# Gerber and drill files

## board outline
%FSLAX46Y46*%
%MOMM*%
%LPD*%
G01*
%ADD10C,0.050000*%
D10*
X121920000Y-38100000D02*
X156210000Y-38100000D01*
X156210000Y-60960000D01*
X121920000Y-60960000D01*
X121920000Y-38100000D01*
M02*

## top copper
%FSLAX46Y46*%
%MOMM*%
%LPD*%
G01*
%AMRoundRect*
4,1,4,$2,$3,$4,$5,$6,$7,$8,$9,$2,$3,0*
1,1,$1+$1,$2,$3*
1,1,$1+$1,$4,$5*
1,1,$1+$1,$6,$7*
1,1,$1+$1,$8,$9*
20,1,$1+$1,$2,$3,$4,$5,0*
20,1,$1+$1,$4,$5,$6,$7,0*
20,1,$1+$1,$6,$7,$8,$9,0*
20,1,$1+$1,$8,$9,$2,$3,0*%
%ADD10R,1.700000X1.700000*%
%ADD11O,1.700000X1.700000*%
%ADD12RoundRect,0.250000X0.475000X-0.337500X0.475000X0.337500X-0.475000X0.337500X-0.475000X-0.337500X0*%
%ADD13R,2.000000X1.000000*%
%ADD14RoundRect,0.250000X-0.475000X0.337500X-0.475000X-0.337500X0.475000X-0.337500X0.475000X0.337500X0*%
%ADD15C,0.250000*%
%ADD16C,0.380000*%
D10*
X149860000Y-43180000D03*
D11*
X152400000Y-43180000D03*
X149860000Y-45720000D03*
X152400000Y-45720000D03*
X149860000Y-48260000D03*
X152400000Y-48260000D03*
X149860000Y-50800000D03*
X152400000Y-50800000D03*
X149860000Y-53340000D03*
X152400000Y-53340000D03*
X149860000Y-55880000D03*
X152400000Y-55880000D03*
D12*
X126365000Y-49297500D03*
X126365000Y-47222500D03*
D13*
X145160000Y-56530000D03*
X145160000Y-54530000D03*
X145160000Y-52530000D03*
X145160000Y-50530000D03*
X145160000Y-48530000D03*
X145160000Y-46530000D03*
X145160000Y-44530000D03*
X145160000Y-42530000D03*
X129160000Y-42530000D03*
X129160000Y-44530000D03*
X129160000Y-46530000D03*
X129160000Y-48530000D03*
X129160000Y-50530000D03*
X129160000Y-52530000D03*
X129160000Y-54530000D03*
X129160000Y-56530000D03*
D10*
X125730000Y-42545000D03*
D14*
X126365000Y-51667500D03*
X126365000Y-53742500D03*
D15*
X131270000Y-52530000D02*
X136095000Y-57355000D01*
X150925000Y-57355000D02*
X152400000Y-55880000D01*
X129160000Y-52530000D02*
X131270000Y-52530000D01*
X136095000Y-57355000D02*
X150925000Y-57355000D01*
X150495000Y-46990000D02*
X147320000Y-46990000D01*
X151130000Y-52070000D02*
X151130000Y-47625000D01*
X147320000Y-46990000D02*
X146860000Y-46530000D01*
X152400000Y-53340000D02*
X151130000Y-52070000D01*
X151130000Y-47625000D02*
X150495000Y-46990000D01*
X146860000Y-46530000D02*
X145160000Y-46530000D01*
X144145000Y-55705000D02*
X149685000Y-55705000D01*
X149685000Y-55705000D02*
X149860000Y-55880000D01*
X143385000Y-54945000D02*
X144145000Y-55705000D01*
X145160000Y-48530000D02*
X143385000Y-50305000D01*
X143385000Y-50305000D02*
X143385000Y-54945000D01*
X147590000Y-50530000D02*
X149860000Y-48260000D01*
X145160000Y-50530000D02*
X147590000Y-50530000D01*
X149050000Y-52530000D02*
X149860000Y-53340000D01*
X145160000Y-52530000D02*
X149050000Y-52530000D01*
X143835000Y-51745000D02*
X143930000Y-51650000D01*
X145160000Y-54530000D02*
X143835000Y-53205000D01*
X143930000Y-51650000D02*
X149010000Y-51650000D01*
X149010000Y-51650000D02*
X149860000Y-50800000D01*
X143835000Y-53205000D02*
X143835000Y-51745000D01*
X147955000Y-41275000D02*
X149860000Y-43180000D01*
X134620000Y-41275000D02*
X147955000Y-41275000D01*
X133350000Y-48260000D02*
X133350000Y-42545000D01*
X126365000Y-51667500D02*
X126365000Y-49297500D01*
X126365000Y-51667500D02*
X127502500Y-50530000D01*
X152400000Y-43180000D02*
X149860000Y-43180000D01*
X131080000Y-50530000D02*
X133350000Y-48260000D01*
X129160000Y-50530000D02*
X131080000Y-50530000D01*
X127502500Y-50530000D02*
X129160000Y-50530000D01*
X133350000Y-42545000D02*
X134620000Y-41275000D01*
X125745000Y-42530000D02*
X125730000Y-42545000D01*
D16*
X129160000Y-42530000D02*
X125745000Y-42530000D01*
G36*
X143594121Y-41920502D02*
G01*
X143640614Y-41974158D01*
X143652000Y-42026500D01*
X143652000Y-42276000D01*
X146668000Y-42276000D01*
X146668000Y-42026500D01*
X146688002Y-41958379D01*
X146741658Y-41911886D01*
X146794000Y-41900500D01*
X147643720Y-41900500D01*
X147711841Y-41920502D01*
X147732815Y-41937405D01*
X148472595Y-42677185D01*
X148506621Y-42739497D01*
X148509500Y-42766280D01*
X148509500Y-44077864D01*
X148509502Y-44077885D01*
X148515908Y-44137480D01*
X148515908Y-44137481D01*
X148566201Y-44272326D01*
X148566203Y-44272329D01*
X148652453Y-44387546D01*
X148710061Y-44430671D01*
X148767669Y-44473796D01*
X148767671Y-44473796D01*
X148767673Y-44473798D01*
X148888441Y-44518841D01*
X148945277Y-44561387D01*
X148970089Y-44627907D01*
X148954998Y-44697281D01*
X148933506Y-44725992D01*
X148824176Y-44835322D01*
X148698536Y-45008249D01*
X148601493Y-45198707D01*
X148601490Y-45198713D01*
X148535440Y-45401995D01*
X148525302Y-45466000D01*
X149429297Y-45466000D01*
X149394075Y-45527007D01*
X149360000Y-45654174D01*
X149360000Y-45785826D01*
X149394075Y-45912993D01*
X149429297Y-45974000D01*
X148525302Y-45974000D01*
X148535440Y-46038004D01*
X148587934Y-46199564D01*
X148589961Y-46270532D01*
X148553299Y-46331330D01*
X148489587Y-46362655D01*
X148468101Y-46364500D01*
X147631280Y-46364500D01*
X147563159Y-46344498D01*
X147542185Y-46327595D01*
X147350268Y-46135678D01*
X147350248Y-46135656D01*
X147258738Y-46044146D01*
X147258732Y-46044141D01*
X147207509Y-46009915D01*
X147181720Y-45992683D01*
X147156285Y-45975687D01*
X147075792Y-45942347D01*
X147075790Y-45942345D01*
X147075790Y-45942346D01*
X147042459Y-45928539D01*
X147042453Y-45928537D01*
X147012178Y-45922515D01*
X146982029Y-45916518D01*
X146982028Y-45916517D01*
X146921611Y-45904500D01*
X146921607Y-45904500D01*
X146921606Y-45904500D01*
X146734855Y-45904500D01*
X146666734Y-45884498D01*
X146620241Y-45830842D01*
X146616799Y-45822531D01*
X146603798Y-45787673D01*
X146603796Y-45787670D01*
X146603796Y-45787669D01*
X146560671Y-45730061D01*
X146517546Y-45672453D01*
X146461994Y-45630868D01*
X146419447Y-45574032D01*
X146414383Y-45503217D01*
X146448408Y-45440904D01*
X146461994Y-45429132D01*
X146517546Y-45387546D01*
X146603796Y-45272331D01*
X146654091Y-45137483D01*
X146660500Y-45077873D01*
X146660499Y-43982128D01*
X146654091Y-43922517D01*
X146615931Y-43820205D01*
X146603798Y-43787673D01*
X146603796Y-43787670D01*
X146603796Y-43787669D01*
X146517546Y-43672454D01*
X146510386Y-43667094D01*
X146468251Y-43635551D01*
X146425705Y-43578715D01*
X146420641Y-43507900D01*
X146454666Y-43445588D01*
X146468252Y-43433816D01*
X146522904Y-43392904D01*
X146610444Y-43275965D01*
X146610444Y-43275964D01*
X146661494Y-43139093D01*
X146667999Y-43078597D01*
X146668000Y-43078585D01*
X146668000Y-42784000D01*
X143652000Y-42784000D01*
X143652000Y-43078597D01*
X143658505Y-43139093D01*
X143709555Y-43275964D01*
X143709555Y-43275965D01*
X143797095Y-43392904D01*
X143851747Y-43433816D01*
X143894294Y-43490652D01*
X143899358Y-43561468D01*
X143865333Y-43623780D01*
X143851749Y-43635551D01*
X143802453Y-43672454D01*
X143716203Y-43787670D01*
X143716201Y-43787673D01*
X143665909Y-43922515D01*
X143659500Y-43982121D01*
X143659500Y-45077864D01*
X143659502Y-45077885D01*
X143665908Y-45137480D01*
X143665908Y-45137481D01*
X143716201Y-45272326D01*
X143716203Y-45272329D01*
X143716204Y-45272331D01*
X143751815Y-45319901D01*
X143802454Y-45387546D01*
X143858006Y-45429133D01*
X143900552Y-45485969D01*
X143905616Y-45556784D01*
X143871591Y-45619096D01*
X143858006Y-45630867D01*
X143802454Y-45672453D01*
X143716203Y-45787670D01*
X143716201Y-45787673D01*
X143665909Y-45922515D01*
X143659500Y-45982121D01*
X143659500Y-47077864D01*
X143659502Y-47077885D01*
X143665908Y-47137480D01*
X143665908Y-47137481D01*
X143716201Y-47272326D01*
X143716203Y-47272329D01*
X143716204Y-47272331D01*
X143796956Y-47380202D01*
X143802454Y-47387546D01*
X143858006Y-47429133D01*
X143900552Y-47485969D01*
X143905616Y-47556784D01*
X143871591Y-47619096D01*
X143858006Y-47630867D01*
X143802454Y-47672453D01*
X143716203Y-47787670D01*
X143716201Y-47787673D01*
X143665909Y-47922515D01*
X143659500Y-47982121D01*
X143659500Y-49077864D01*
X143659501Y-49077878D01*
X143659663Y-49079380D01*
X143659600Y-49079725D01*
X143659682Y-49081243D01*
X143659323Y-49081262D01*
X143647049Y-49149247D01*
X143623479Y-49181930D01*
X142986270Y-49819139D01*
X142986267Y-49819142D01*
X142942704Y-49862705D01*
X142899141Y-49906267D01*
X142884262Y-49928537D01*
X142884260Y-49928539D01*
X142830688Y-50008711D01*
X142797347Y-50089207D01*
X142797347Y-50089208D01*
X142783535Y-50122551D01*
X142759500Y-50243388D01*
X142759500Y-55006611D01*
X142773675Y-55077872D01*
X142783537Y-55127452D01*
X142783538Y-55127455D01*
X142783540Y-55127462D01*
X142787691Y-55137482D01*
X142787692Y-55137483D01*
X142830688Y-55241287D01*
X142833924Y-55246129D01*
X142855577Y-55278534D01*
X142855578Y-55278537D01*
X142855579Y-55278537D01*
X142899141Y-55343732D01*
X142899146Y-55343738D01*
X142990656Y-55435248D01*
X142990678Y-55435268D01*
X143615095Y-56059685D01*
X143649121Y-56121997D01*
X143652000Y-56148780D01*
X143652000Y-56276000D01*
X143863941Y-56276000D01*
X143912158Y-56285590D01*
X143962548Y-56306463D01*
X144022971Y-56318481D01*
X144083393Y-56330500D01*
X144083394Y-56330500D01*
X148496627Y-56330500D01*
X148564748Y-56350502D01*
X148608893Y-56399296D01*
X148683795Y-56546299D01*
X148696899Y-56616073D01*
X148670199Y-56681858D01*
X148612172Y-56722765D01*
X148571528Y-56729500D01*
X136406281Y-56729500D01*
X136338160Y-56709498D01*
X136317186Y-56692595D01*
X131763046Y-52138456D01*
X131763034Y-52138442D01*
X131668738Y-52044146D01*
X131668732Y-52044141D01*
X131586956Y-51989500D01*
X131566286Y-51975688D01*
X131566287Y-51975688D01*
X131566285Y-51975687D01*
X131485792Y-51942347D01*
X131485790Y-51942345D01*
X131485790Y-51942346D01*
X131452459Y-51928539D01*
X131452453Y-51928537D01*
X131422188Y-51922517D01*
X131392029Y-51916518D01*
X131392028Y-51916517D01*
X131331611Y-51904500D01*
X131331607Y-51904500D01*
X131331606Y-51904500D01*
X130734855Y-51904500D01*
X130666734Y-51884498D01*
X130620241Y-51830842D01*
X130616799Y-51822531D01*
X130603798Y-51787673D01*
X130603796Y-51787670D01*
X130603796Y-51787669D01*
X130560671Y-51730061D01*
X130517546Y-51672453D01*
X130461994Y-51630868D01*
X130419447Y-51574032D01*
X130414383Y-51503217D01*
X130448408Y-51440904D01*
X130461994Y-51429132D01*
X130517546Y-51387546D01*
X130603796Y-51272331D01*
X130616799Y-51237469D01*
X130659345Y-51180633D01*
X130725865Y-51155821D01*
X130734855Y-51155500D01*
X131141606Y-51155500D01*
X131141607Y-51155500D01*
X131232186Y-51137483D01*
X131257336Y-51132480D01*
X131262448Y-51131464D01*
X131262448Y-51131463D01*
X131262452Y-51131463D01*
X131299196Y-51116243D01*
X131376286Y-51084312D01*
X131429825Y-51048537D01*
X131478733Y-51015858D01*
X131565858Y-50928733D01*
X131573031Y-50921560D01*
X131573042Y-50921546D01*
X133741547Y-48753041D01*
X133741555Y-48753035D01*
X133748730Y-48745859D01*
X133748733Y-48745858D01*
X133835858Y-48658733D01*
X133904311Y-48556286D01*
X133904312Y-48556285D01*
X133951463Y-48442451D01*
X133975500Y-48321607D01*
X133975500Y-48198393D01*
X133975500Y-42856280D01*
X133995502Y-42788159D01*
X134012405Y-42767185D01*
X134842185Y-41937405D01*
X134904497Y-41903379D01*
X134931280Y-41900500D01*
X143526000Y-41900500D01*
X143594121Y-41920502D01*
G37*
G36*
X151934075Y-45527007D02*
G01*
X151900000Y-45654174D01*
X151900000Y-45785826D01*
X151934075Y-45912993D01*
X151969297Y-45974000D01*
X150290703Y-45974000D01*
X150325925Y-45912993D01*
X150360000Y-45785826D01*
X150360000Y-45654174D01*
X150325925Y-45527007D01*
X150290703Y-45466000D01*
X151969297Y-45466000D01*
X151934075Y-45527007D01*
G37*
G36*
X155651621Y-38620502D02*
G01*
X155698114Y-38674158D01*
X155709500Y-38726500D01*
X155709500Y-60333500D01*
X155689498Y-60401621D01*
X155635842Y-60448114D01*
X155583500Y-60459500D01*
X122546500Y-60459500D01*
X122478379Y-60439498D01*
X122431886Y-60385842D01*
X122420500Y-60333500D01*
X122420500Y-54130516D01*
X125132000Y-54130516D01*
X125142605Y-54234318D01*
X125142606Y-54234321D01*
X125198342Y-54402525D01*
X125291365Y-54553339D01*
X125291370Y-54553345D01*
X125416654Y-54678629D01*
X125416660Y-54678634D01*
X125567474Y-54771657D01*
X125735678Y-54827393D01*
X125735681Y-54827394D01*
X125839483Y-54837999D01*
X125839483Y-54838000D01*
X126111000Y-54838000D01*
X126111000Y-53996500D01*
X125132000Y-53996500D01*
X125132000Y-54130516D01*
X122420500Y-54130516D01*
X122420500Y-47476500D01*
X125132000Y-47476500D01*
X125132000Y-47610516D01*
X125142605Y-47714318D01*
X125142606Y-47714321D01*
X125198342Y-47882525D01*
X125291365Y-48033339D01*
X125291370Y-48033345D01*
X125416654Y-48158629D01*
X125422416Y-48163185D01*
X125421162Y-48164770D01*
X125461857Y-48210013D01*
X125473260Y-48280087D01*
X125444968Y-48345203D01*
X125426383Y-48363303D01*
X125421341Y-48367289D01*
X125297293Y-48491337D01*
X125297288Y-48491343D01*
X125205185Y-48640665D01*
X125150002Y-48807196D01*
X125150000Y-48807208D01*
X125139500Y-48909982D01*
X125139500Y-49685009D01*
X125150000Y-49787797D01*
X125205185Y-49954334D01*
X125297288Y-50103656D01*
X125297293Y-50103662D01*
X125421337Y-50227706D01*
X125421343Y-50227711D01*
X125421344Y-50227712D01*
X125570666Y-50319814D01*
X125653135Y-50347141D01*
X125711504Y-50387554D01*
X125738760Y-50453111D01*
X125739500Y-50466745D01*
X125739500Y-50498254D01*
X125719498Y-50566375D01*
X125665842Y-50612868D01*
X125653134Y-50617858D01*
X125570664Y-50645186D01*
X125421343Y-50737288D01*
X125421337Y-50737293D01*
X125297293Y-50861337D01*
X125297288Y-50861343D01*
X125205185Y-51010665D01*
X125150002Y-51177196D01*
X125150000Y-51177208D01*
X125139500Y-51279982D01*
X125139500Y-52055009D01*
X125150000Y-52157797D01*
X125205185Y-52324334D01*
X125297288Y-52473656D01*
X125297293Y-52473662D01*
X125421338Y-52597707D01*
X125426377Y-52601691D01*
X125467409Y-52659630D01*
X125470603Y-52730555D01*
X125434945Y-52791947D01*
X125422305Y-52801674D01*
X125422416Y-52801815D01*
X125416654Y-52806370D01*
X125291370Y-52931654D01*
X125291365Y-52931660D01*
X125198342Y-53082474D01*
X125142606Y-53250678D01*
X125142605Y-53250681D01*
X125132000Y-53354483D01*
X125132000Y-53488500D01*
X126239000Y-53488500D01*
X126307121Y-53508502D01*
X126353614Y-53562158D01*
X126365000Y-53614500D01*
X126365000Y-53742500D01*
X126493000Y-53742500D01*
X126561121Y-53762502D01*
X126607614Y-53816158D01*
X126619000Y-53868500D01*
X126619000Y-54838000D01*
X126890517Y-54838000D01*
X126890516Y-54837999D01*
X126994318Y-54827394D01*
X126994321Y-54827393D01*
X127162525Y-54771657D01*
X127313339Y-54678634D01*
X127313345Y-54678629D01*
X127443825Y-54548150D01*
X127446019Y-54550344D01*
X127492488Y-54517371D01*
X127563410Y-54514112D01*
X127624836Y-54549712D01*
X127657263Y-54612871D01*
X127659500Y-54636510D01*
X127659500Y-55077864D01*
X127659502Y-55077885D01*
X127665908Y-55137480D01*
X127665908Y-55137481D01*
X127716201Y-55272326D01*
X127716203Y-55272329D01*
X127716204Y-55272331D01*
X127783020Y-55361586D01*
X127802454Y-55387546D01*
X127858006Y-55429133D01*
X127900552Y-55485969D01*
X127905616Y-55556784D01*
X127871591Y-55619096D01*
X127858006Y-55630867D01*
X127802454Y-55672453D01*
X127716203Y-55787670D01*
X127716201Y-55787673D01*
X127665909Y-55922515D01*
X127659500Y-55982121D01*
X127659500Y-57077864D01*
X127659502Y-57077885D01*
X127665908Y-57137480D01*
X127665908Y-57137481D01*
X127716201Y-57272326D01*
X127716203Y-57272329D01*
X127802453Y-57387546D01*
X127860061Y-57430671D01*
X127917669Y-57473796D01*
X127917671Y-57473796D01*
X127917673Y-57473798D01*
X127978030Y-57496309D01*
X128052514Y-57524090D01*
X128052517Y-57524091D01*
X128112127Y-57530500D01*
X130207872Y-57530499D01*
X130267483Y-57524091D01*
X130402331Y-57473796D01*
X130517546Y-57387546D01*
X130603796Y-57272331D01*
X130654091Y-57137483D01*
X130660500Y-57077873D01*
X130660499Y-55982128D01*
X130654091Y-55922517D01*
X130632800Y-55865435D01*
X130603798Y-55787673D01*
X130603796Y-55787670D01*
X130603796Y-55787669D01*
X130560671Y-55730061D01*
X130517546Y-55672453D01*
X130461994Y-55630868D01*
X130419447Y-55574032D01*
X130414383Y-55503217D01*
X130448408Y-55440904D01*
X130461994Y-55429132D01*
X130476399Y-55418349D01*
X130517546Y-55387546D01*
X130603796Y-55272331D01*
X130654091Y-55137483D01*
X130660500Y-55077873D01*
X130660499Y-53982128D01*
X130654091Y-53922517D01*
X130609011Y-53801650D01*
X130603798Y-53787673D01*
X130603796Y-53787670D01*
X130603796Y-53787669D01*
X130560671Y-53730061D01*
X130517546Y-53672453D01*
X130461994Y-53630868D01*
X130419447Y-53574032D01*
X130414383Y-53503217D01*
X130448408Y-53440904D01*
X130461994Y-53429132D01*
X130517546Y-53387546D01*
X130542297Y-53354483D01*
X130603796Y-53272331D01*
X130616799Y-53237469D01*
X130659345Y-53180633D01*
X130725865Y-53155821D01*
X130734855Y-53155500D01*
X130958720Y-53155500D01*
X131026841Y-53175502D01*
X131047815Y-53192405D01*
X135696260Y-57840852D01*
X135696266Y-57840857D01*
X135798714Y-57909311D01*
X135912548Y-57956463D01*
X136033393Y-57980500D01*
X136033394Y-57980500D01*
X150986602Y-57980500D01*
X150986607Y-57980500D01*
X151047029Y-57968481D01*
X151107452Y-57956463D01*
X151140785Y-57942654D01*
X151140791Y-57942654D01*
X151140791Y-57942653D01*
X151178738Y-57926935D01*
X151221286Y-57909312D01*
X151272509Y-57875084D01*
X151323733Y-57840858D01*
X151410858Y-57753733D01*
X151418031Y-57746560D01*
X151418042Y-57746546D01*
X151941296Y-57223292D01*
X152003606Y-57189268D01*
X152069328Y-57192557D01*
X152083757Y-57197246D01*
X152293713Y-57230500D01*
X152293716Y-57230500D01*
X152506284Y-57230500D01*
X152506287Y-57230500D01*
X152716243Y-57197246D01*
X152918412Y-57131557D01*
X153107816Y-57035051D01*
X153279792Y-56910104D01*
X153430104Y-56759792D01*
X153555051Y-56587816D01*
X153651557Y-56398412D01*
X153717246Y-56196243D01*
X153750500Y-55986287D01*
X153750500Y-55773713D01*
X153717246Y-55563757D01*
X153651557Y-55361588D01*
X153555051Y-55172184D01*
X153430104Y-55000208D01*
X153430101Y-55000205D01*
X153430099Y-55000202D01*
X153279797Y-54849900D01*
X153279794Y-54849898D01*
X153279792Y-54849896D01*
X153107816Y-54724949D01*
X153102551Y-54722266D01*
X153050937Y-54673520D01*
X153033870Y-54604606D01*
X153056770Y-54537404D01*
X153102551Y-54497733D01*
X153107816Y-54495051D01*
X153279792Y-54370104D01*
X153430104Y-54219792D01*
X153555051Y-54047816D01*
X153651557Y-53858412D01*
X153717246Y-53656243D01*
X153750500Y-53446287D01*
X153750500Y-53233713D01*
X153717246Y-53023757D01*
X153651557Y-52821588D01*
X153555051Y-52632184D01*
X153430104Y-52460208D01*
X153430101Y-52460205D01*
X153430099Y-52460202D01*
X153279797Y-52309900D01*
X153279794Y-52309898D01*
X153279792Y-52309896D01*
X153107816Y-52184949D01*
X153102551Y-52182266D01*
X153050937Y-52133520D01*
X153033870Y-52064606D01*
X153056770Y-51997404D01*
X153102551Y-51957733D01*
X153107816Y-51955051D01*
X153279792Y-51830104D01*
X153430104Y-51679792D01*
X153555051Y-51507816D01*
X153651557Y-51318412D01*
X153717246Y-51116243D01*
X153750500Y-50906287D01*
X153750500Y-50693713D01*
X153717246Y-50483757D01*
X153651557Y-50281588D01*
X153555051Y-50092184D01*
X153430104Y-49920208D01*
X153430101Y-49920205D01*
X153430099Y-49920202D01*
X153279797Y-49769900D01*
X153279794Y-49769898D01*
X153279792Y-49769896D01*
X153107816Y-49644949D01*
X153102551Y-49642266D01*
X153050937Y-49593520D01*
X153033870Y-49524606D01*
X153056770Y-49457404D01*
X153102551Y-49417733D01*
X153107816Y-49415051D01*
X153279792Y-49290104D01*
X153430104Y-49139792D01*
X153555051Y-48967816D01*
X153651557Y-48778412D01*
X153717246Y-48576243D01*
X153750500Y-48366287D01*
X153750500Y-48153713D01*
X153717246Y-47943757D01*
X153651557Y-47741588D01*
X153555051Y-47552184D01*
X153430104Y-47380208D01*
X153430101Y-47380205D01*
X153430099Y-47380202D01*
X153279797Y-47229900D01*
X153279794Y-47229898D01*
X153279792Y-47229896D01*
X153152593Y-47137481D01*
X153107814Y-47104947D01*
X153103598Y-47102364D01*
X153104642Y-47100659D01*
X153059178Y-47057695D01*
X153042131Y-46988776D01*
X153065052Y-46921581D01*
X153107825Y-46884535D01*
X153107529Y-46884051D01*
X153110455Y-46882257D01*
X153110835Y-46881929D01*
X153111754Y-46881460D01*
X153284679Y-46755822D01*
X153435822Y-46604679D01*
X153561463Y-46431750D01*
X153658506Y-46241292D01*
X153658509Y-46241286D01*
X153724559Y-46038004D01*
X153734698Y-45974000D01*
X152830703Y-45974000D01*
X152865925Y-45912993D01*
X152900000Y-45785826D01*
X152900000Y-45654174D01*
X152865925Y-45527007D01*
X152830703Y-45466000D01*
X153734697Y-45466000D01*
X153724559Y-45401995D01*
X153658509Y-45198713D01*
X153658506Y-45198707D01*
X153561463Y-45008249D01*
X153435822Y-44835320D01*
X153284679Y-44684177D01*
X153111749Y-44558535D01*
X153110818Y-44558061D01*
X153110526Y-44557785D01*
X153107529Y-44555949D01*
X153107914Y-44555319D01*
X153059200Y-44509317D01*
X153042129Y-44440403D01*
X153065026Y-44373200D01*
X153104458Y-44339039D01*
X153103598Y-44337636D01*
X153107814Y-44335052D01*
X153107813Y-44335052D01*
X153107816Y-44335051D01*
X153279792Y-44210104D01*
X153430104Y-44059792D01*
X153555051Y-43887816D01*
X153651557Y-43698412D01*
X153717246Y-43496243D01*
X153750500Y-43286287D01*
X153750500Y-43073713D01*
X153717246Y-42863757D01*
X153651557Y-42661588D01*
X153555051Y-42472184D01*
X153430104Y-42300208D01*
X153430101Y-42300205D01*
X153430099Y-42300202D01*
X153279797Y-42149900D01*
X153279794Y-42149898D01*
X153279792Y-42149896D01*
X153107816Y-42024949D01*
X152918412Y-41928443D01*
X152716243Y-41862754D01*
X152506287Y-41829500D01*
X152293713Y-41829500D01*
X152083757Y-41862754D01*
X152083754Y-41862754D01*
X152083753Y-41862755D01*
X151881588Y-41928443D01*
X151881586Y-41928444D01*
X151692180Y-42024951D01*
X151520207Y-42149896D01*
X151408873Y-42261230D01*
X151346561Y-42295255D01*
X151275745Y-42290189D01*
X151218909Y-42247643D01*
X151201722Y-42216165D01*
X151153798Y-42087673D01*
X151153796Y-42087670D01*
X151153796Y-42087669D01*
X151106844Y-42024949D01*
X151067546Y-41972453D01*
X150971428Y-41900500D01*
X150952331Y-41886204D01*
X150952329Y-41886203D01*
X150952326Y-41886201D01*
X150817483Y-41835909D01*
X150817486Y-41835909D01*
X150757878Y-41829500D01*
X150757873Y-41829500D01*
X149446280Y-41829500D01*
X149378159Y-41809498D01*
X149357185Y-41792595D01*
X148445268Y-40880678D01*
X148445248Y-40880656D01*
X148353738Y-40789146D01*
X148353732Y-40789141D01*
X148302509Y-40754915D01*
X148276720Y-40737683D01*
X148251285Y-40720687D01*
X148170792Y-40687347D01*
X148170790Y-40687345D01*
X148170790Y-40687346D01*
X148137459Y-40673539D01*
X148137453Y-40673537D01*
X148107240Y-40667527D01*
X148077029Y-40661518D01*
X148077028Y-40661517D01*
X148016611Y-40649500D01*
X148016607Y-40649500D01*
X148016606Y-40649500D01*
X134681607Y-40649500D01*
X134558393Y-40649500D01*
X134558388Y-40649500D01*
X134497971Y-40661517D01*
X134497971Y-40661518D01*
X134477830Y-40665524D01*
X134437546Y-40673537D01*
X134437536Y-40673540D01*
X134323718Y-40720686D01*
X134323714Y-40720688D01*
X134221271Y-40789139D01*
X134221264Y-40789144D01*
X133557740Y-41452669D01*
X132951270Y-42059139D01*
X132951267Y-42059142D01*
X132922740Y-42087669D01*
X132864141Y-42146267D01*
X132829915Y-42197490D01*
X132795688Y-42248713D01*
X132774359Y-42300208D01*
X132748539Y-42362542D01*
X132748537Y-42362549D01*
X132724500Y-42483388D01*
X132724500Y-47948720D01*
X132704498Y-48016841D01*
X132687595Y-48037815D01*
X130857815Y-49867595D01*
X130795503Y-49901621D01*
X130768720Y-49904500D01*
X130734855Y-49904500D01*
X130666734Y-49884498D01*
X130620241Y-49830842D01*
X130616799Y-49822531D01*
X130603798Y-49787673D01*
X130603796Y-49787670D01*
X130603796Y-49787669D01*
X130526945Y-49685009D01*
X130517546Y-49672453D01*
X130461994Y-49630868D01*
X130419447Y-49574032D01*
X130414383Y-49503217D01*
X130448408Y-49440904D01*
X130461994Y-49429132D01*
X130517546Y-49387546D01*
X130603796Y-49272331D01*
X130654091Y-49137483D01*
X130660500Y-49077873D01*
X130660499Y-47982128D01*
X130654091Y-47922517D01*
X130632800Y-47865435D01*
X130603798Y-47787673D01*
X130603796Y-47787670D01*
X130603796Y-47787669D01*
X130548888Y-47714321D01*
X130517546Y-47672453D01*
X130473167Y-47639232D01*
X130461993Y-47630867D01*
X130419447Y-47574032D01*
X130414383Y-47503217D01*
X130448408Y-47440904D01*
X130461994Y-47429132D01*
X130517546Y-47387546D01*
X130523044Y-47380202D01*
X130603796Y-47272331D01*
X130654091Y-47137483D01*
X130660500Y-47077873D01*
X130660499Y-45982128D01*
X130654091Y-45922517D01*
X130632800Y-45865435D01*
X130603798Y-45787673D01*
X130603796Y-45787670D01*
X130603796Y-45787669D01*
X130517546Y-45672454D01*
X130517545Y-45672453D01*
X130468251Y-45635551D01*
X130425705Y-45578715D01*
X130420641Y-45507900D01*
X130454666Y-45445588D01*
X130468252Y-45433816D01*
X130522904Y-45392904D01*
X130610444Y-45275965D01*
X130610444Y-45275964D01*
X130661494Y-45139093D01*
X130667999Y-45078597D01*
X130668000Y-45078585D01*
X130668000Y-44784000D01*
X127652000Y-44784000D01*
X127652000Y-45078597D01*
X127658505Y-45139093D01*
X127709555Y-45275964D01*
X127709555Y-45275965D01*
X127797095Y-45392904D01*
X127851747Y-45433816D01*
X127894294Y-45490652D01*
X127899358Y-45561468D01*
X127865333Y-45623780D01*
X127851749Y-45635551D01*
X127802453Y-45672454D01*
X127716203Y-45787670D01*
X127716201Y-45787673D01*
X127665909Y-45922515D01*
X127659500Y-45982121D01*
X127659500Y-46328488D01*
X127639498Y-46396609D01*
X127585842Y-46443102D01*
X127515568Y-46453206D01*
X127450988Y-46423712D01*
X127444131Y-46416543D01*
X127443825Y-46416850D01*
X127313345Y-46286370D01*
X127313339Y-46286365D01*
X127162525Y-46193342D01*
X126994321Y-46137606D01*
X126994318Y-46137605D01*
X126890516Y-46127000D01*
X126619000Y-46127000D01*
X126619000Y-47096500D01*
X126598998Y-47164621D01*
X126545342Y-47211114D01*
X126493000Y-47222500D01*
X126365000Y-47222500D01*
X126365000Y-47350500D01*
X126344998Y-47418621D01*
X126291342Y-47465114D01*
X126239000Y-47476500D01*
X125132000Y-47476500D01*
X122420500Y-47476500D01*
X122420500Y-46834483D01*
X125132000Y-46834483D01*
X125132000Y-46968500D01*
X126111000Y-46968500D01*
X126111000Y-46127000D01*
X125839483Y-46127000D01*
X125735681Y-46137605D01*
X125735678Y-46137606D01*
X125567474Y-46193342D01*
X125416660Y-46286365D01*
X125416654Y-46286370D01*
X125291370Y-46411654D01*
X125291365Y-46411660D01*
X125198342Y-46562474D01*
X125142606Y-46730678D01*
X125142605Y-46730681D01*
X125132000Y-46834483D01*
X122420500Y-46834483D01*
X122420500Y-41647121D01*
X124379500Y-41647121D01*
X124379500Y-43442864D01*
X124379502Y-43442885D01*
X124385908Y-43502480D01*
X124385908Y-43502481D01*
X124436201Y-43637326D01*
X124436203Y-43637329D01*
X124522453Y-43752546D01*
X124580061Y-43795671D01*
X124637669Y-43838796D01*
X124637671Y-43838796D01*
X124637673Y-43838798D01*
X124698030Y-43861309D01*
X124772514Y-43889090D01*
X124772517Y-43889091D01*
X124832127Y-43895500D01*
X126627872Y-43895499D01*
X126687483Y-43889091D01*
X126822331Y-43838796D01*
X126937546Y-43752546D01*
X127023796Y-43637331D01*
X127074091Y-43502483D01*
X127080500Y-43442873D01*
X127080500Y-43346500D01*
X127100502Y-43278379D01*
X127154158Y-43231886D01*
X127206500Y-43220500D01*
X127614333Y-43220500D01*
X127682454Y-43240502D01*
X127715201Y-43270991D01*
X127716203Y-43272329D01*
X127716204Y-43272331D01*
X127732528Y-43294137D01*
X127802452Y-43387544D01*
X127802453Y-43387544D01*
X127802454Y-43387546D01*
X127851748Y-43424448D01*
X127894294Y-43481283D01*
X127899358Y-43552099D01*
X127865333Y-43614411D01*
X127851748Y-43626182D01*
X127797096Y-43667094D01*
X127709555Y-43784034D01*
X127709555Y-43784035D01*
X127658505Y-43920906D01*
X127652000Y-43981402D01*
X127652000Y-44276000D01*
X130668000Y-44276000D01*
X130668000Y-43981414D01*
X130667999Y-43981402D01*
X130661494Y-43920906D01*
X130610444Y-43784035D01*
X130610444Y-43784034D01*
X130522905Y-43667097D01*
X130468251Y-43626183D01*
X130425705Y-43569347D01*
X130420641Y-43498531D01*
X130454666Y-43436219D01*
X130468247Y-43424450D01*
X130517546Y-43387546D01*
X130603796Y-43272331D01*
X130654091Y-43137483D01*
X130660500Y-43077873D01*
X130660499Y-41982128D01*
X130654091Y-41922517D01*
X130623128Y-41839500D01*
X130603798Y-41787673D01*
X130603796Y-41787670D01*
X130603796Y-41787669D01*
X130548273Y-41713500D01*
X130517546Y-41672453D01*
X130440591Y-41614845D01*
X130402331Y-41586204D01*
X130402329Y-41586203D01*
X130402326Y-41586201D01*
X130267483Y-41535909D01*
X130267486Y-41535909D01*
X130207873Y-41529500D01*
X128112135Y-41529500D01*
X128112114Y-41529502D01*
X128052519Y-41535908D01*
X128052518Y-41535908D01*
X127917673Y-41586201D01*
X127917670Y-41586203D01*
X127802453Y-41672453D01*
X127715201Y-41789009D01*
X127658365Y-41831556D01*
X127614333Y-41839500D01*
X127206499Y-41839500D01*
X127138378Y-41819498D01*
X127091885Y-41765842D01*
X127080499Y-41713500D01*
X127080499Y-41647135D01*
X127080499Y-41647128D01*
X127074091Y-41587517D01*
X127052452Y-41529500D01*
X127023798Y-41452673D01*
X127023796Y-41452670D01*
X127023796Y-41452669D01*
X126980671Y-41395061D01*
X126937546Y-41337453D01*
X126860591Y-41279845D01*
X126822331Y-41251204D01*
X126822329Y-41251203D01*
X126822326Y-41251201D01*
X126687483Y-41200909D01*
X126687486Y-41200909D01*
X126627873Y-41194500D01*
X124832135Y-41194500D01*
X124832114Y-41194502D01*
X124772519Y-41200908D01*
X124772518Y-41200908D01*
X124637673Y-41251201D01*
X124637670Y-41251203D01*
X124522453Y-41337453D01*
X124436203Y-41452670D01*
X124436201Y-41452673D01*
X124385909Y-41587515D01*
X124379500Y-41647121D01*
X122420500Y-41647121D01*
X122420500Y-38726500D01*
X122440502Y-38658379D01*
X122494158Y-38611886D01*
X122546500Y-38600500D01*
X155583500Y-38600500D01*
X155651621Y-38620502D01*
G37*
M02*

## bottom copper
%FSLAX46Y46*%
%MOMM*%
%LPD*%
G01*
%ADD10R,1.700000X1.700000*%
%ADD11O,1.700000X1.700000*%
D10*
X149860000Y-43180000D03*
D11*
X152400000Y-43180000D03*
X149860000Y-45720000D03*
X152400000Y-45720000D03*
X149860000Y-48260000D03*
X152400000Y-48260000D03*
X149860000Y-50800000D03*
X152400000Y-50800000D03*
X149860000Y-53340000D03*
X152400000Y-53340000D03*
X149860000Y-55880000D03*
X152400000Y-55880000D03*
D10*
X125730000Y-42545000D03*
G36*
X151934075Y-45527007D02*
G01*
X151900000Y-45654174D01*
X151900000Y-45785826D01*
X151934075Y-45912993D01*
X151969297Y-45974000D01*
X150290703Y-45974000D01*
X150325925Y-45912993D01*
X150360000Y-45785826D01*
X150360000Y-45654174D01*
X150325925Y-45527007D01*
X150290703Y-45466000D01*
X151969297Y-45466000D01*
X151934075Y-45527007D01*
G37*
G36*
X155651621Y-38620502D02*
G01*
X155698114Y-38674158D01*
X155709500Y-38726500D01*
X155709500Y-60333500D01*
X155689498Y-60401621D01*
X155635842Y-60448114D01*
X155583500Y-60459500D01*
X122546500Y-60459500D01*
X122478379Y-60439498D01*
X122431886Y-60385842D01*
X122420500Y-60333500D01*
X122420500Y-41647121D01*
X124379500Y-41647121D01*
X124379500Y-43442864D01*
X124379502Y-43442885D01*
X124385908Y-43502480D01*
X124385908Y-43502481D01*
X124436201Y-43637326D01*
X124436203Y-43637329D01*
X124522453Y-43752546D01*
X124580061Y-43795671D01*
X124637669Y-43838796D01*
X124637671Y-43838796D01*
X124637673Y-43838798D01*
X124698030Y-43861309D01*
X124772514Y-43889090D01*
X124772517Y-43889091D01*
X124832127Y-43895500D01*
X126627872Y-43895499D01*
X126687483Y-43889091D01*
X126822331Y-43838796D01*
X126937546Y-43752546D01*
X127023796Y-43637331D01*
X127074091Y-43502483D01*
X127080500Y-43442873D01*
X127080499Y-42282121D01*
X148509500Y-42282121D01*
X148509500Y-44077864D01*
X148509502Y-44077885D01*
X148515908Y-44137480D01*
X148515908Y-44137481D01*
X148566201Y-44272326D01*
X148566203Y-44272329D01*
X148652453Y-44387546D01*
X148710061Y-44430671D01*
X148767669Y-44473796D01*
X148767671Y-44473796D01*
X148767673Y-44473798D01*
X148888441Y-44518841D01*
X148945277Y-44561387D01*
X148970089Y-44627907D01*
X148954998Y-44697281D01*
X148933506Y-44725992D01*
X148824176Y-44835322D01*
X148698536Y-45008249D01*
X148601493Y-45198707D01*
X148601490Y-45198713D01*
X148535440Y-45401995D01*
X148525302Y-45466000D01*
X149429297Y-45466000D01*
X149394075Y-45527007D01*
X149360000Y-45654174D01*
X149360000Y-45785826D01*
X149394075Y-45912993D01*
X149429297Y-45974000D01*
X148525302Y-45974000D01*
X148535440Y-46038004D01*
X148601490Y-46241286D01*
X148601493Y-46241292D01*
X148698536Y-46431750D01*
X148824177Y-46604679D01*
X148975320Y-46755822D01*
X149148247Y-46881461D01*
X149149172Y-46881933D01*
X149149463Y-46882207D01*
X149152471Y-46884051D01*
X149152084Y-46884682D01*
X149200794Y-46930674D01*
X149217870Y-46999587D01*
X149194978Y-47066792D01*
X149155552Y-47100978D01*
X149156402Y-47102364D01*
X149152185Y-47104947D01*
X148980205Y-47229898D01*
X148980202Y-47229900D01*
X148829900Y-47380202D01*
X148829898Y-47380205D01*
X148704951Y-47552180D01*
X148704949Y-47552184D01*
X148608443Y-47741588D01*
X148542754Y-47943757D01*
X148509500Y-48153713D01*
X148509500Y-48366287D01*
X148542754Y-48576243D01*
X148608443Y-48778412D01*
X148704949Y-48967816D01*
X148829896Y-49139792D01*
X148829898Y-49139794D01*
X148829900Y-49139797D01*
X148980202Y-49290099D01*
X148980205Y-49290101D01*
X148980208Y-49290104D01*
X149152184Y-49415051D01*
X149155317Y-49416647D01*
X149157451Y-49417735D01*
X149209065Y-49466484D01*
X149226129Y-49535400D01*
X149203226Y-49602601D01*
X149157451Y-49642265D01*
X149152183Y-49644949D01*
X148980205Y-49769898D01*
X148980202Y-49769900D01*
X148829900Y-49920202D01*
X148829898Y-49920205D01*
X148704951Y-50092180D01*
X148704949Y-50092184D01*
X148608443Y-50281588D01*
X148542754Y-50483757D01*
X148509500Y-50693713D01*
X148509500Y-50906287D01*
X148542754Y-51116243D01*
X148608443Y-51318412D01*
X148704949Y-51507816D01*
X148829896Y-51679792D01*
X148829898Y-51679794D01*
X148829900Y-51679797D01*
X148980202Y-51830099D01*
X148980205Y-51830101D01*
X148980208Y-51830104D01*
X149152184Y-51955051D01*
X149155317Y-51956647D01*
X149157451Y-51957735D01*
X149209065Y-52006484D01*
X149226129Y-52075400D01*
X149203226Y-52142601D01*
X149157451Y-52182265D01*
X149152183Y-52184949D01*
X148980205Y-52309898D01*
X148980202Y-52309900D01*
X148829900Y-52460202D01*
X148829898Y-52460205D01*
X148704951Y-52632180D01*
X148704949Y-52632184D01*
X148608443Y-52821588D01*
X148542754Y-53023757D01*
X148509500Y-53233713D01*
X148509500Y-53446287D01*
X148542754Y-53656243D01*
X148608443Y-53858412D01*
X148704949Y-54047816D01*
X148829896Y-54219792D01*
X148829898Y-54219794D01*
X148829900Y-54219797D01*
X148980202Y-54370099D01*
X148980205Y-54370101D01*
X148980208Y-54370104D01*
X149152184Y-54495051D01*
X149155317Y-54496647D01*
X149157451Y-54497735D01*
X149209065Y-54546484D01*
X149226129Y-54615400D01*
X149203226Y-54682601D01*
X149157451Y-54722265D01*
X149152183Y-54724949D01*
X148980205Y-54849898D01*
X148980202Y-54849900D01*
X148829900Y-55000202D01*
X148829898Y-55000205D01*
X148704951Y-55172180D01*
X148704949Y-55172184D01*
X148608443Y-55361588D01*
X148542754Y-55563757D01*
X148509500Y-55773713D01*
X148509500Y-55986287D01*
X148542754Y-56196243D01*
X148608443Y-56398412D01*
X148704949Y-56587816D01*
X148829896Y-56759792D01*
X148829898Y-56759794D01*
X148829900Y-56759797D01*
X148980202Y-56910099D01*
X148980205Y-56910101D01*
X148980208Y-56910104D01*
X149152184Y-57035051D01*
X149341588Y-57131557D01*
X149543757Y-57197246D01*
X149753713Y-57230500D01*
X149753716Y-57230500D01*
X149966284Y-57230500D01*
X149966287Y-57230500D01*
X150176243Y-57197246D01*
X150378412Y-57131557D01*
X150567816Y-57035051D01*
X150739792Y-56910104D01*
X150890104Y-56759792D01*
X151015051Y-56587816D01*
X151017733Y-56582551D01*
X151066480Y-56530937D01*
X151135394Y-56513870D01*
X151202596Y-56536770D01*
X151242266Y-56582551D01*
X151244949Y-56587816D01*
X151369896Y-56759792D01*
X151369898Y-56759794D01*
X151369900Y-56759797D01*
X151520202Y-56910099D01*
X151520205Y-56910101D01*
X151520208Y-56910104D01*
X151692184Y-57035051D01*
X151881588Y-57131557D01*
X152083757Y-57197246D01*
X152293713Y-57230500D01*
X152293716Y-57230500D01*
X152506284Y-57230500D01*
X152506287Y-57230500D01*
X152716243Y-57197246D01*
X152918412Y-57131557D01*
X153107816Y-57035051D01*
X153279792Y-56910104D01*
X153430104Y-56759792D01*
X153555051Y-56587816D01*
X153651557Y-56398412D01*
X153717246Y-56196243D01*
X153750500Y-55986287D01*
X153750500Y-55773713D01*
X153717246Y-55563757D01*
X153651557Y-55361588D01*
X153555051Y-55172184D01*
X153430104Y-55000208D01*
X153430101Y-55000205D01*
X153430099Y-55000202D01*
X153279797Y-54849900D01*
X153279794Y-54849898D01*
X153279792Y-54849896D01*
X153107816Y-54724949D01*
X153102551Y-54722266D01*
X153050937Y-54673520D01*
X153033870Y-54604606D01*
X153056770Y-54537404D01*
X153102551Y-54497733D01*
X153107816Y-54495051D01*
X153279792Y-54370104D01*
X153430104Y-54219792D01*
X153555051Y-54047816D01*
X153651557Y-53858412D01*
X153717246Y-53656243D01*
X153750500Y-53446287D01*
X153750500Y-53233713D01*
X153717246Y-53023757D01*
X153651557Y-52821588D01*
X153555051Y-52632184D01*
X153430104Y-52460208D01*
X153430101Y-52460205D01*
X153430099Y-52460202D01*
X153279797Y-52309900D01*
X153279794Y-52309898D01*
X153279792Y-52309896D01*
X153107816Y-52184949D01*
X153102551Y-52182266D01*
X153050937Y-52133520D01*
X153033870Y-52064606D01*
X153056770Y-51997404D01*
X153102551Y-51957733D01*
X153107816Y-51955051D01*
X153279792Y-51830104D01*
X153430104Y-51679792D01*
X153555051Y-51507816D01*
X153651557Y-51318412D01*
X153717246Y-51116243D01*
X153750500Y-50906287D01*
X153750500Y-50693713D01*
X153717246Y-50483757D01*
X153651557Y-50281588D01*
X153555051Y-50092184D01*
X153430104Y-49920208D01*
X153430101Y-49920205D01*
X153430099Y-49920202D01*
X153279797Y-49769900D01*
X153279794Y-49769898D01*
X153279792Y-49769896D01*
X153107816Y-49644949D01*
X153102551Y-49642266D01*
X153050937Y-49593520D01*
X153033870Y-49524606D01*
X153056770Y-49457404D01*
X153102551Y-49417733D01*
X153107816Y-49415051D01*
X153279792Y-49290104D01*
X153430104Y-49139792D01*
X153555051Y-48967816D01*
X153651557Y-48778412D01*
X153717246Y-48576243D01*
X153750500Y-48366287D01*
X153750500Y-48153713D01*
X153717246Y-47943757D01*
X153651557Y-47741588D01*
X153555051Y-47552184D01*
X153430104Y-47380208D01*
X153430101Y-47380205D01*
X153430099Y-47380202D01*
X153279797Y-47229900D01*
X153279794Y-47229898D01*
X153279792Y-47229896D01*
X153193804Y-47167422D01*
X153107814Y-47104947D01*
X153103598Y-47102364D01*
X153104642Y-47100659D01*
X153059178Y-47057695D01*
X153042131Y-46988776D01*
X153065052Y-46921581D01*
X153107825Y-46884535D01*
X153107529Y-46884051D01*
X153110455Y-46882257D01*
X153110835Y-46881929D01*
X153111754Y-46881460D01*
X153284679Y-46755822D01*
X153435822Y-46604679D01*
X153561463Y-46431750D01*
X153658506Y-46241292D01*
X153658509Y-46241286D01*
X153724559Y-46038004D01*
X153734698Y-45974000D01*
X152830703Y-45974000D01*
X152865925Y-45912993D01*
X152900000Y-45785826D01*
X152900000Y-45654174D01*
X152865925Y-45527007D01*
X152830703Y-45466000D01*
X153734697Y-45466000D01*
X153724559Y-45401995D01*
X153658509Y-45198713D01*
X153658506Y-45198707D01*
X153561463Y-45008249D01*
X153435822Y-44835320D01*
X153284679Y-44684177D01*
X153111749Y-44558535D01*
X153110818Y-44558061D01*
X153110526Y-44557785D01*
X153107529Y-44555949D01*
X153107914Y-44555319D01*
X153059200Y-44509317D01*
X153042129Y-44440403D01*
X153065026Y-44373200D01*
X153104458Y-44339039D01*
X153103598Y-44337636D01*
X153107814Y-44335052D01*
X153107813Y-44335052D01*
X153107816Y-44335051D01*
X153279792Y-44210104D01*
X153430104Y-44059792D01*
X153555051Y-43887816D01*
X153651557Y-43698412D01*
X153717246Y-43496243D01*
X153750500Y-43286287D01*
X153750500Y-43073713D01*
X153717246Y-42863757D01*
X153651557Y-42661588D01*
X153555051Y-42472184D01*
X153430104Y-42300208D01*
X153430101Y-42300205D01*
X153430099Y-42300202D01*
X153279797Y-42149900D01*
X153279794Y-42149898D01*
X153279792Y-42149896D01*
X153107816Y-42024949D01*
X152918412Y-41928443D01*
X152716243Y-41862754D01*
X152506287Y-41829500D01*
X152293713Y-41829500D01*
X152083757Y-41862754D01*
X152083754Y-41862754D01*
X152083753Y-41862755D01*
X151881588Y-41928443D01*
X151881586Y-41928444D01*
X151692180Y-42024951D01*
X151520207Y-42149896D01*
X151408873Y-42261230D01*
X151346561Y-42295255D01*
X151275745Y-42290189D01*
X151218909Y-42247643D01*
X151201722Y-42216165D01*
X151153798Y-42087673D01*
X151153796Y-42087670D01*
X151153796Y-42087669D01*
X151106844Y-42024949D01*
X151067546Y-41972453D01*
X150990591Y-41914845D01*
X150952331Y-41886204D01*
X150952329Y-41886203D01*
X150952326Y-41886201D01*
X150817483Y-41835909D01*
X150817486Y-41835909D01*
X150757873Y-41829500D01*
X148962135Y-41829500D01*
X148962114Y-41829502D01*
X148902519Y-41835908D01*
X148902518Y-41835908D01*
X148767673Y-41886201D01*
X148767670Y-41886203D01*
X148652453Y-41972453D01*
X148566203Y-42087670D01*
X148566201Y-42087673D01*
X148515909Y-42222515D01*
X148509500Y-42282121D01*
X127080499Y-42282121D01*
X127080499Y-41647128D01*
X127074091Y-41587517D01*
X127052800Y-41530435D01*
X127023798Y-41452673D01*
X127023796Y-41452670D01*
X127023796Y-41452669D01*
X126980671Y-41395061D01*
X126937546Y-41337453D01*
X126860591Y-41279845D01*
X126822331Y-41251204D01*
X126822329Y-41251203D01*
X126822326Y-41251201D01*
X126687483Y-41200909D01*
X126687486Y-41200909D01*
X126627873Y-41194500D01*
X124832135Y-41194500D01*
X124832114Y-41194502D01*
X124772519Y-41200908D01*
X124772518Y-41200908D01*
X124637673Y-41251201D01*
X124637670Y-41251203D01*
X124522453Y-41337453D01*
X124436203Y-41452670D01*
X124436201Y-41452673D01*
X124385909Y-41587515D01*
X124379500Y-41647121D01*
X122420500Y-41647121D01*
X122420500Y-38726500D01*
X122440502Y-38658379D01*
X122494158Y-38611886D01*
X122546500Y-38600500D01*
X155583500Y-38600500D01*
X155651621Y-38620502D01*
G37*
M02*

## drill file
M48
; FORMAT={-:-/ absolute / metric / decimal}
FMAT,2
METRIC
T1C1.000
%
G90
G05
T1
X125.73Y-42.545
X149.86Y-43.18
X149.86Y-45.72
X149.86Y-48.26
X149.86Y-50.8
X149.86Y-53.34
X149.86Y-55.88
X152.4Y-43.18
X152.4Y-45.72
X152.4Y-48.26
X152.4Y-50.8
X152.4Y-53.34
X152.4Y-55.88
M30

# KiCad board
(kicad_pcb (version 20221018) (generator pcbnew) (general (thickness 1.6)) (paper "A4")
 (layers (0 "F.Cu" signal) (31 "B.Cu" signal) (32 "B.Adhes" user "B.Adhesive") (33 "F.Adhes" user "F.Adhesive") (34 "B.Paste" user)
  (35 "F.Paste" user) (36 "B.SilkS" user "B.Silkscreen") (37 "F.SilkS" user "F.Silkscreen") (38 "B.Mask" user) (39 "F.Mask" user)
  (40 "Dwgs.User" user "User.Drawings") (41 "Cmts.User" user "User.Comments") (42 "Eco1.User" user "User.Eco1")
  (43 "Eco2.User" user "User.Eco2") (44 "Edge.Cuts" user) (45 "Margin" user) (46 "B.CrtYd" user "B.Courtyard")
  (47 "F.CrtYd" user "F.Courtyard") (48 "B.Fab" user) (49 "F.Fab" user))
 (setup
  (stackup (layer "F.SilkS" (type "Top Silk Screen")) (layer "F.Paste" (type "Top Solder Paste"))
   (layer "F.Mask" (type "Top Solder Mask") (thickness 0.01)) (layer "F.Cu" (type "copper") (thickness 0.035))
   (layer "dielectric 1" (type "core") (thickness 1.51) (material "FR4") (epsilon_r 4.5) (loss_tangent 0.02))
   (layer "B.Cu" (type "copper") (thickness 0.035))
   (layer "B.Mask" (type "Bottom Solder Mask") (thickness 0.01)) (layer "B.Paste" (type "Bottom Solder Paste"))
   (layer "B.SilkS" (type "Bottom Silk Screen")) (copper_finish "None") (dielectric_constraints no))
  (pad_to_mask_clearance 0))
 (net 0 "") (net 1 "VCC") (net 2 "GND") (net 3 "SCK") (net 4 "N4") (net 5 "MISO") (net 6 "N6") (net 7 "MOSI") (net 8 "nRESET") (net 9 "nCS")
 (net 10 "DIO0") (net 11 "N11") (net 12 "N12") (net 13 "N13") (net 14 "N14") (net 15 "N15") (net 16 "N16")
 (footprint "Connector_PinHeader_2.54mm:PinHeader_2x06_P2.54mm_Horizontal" (layer "F.Cu") (at 149.86 43.18)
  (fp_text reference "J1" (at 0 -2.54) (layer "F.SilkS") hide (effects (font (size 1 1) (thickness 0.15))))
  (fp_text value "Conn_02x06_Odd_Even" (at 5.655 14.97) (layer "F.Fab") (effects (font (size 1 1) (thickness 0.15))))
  (pad "1" thru_hole rect (at 0 0) (size 1.7 1.7) (drill 1) (layers "*.Cu" "*.Mask") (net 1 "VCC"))
  (pad "2" thru_hole oval (at 2.54 0) (size 1.7 1.7) (drill 1) (layers "*.Cu" "*.Mask") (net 1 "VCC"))
  (pad "3" thru_hole oval (at 0 2.54) (size 1.7 1.7) (drill 1) (layers "*.Cu" "*.Mask") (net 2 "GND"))
  (pad "4" thru_hole oval (at 2.54 2.54) (size 1.7 1.7) (drill 1) (layers "*.Cu" "*.Mask") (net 2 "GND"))
  (pad "5" thru_hole oval (at 0 5.08) (size 1.7 1.7) (drill 1) (layers "*.Cu" "*.Mask") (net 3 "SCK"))
  (pad "6" thru_hole oval (at 2.54 5.08) (size 1.7 1.7) (drill 1) (layers "*.Cu" "*.Mask") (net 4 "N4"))
  (pad "7" thru_hole oval (at 0 7.62) (size 1.7 1.7) (drill 1) (layers "*.Cu" "*.Mask") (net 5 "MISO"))
  (pad "8" thru_hole oval (at 2.54 7.62) (size 1.7 1.7) (drill 1) (layers "*.Cu" "*.Mask") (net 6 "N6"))
  (pad "9" thru_hole oval (at 0 10.16) (size 1.7 1.7) (drill 1) (layers "*.Cu" "*.Mask") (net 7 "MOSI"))
  (pad "10" thru_hole oval (at 2.54 10.16) (size 1.7 1.7) (drill 1) (layers "*.Cu" "*.Mask") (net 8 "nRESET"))
  (pad "11" thru_hole oval (at 0 12.7) (size 1.7 1.7) (drill 1) (layers "*.Cu" "*.Mask") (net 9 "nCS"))
  (pad "12" thru_hole oval (at 2.54 12.7) (size 1.7 1.7) (drill 1) (layers "*.Cu" "*.Mask") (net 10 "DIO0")))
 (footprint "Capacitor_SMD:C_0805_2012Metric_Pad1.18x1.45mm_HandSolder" (layer "F.Cu") (at 126.365 48.26 90)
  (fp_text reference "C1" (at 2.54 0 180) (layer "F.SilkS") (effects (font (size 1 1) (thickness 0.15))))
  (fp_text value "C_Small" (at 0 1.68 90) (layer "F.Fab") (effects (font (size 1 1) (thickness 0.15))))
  (pad "1" smd roundrect (at -1.0375 0 90) (size 1.175 1.45) (layers "F.Cu" "F.Paste" "F.Mask") (roundrect_rratio 0.2127659574)
   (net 1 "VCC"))
  (pad "2" smd roundrect (at 1.0375 0 90) (size 1.175 1.45) (layers "F.Cu" "F.Paste" "F.Mask") (roundrect_rratio 0.2127659574) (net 2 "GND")))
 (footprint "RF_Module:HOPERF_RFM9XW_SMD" (layer "F.Cu") (at 137.16 49.53 180)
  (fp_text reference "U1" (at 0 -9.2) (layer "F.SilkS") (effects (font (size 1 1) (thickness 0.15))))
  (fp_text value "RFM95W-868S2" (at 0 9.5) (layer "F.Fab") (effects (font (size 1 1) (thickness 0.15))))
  (pad "1" smd rect (at -8 -7 180) (size 2 1) (layers "F.Cu" "F.Paste" "F.Mask") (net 2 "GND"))
  (pad "2" smd rect (at -8 -5 180) (size 2 1) (layers "F.Cu" "F.Paste" "F.Mask") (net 5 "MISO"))
  (pad "3" smd rect (at -8 -3 180) (size 2 1) (layers "F.Cu" "F.Paste" "F.Mask") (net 7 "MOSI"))
  (pad "4" smd rect (at -8 -1 180) (size 2 1) (layers "F.Cu" "F.Paste" "F.Mask") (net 3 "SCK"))
  (pad "5" smd rect (at -8 1 180) (size 2 1) (layers "F.Cu" "F.Paste" "F.Mask") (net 9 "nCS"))
  (pad "6" smd rect (at -8 3 180) (size 2 1) (layers "F.Cu" "F.Paste" "F.Mask") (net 8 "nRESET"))
  (pad "7" smd rect (at -8 5 180) (size 2 1) (layers "F.Cu" "F.Paste" "F.Mask") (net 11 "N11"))
  (pad "8" smd rect (at -8 7 180) (size 2 1) (layers "F.Cu" "F.Paste" "F.Mask") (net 2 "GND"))
  (pad "9" smd rect (at 8 7 180) (size 2 1) (layers "F.Cu" "F.Paste" "F.Mask") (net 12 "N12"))
  (pad "10" smd rect (at 8 5 180) (size 2 1) (layers "F.Cu" "F.Paste" "F.Mask") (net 2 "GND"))
  (pad "11" smd rect (at 8 3 180) (size 2 1) (layers "F.Cu" "F.Paste" "F.Mask") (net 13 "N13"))
  (pad "12" smd rect (at 8 1 180) (size 2 1) (layers "F.Cu" "F.Paste" "F.Mask") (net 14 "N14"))
  (pad "13" smd rect (at 8 -1 180) (size 2 1) (layers "F.Cu" "F.Paste" "F.Mask") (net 1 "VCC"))
  (pad "14" smd rect (at 8 -3 180) (size 2 1) (layers "F.Cu" "F.Paste" "F.Mask") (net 10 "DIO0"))
  (pad "15" smd rect (at 8 -5 180) (size 2 1) (layers "F.Cu" "F.Paste" "F.Mask") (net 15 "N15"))
  (pad "16" smd rect (at 8 -7 180) (size 2 1) (layers "F.Cu" "F.Paste" "F.Mask") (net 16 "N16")))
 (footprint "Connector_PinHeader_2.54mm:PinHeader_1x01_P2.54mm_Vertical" (layer "F.Cu") (at 125.73 42.545)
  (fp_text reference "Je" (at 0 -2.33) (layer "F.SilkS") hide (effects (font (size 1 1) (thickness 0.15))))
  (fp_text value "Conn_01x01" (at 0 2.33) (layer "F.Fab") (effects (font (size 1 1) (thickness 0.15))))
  (pad "1" thru_hole rect (at 0 0) (size 1.7 1.7) (drill 1) (layers "*.Cu" "*.Mask") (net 12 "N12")))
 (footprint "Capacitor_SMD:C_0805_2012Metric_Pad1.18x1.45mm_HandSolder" (layer "F.Cu") (at 126.365 52.705 -90)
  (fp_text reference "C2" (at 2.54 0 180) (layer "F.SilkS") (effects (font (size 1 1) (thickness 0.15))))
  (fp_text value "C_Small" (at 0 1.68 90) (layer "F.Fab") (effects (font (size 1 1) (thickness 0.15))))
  (pad "1" smd roundrect (at -1.0375 0 270) (size 1.175 1.45) (layers "F.Cu" "F.Paste" "F.Mask") (roundrect_rratio 0.2127659574)
   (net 1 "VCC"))
  (pad "2" smd roundrect (at 1.0375 0 270) (size 1.175 1.45) (layers "F.Cu" "F.Paste" "F.Mask") (roundrect_rratio 0.2127659574)
   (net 2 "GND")))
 (gr_rect (start 121.92 38.1) (end 156.21 60.96) (stroke (width 0.05) (type solid)) (fill none) (layer "Edge.Cuts"))
 (segment (start 131.27 52.53) (end 136.095 57.355) (width 0.25) (layer "F.Cu") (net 10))
 (segment (start 150.925 57.355) (end 152.4 55.88) (width 0.25) (layer "F.Cu") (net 10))
 (segment (start 129.16 52.53) (end 131.27 52.53) (width 0.25) (layer "F.Cu") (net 10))
 (segment (start 136.095 57.355) (end 150.925 57.355) (width 0.25) (layer "F.Cu") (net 10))
 (segment (start 150.495 46.99) (end 147.32 46.99) (width 0.25) (layer "F.Cu") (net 8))
 (segment (start 151.13 52.07) (end 151.13 47.625) (width 0.25) (layer "F.Cu") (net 8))
 (segment (start 147.32 46.99) (end 146.86 46.53) (width 0.25) (layer "F.Cu") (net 8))
 (segment (start 152.4 53.34) (end 151.13 52.07) (width 0.25) (layer "F.Cu") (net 8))
 (segment (start 151.13 47.625) (end 150.495 46.99) (width 0.25) (layer "F.Cu") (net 8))
 (segment (start 146.86 46.53) (end 145.16 46.53) (width 0.25) (layer "F.Cu") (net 8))
 (segment (start 144.145 55.705) (end 149.685 55.705) (width 0.25) (layer "F.Cu") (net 9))
 (segment (start 149.685 55.705) (end 149.86 55.88) (width 0.25) (layer "F.Cu") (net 9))
 (segment (start 143.385 54.945) (end 144.145 55.705) (width 0.25) (layer "F.Cu") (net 9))
 (segment (start 145.16 48.53) (end 143.385 50.305) (width 0.25) (layer "F.Cu") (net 9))
 (segment (start 143.385 50.305) (end 143.385 54.945) (width 0.25) (layer "F.Cu") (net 9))
 (segment (start 147.59 50.53) (end 149.86 48.26) (width 0.25) (layer "F.Cu") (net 3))
 (segment (start 145.16 50.53) (end 147.59 50.53) (width 0.25) (layer "F.Cu") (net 3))
 (segment (start 149.05 52.53) (end 149.86 53.34) (width 0.25) (layer "F.Cu") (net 7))
 (segment (start 145.16 52.53) (end 149.05 52.53) (width 0.25) (layer "F.Cu") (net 7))
 (segment (start 143.835 51.745) (end 143.93 51.65) (width 0.25) (layer "F.Cu") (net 5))
 (segment (start 145.16 54.53) (end 143.835 53.205) (width 0.25) (layer "F.Cu") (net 5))
 (segment (start 143.93 51.65) (end 149.01 51.65) (width 0.25) (layer "F.Cu") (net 5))
 (segment (start 149.01 51.65) (end 149.86 50.8) (width 0.25) (layer "F.Cu") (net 5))
 (segment (start 143.835 53.205) (end 143.835 51.745) (width 0.25) (layer "F.Cu") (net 5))
 (segment (start 147.955 41.275) (end 149.86 43.18) (width 0.25) (layer "F.Cu") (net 1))
 (segment (start 134.62 41.275) (end 147.955 41.275) (width 0.25) (layer "F.Cu") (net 1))
 (segment (start 133.35 48.26) (end 133.35 42.545) (width 0.25) (layer "F.Cu") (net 1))
 (segment (start 126.365 51.6675) (end 126.365 49.2975) (width 0.25) (layer "F.Cu") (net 1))
 (segment (start 126.365 51.6675) (end 127.5025 50.53) (width 0.25) (layer "F.Cu") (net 1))
 (segment (start 152.4 43.18) (end 149.86 43.18) (width 0.25) (layer "F.Cu") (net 1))
 (segment (start 131.08 50.53) (end 133.35 48.26) (width 0.25) (layer "F.Cu") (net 1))
 (segment (start 129.16 50.53) (end 131.08 50.53) (width 0.25) (layer "F.Cu") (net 1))
 (segment (start 127.5025 50.53) (end 129.16 50.53) (width 0.25) (layer "F.Cu") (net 1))
 (segment (start 133.35 42.545) (end 134.62 41.275) (width 0.25) (layer "F.Cu") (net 1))
 (segment (start 125.745 42.53) (end 125.73 42.545) (width 0.25) (layer "F.Cu") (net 12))
 (segment (start 129.16 42.53) (end 125.745 42.53) (width 0.38) (layer "F.Cu") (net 12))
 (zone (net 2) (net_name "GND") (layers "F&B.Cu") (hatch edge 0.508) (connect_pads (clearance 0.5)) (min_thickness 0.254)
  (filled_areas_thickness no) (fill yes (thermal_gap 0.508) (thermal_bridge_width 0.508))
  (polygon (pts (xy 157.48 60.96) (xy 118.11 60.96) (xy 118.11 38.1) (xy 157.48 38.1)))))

